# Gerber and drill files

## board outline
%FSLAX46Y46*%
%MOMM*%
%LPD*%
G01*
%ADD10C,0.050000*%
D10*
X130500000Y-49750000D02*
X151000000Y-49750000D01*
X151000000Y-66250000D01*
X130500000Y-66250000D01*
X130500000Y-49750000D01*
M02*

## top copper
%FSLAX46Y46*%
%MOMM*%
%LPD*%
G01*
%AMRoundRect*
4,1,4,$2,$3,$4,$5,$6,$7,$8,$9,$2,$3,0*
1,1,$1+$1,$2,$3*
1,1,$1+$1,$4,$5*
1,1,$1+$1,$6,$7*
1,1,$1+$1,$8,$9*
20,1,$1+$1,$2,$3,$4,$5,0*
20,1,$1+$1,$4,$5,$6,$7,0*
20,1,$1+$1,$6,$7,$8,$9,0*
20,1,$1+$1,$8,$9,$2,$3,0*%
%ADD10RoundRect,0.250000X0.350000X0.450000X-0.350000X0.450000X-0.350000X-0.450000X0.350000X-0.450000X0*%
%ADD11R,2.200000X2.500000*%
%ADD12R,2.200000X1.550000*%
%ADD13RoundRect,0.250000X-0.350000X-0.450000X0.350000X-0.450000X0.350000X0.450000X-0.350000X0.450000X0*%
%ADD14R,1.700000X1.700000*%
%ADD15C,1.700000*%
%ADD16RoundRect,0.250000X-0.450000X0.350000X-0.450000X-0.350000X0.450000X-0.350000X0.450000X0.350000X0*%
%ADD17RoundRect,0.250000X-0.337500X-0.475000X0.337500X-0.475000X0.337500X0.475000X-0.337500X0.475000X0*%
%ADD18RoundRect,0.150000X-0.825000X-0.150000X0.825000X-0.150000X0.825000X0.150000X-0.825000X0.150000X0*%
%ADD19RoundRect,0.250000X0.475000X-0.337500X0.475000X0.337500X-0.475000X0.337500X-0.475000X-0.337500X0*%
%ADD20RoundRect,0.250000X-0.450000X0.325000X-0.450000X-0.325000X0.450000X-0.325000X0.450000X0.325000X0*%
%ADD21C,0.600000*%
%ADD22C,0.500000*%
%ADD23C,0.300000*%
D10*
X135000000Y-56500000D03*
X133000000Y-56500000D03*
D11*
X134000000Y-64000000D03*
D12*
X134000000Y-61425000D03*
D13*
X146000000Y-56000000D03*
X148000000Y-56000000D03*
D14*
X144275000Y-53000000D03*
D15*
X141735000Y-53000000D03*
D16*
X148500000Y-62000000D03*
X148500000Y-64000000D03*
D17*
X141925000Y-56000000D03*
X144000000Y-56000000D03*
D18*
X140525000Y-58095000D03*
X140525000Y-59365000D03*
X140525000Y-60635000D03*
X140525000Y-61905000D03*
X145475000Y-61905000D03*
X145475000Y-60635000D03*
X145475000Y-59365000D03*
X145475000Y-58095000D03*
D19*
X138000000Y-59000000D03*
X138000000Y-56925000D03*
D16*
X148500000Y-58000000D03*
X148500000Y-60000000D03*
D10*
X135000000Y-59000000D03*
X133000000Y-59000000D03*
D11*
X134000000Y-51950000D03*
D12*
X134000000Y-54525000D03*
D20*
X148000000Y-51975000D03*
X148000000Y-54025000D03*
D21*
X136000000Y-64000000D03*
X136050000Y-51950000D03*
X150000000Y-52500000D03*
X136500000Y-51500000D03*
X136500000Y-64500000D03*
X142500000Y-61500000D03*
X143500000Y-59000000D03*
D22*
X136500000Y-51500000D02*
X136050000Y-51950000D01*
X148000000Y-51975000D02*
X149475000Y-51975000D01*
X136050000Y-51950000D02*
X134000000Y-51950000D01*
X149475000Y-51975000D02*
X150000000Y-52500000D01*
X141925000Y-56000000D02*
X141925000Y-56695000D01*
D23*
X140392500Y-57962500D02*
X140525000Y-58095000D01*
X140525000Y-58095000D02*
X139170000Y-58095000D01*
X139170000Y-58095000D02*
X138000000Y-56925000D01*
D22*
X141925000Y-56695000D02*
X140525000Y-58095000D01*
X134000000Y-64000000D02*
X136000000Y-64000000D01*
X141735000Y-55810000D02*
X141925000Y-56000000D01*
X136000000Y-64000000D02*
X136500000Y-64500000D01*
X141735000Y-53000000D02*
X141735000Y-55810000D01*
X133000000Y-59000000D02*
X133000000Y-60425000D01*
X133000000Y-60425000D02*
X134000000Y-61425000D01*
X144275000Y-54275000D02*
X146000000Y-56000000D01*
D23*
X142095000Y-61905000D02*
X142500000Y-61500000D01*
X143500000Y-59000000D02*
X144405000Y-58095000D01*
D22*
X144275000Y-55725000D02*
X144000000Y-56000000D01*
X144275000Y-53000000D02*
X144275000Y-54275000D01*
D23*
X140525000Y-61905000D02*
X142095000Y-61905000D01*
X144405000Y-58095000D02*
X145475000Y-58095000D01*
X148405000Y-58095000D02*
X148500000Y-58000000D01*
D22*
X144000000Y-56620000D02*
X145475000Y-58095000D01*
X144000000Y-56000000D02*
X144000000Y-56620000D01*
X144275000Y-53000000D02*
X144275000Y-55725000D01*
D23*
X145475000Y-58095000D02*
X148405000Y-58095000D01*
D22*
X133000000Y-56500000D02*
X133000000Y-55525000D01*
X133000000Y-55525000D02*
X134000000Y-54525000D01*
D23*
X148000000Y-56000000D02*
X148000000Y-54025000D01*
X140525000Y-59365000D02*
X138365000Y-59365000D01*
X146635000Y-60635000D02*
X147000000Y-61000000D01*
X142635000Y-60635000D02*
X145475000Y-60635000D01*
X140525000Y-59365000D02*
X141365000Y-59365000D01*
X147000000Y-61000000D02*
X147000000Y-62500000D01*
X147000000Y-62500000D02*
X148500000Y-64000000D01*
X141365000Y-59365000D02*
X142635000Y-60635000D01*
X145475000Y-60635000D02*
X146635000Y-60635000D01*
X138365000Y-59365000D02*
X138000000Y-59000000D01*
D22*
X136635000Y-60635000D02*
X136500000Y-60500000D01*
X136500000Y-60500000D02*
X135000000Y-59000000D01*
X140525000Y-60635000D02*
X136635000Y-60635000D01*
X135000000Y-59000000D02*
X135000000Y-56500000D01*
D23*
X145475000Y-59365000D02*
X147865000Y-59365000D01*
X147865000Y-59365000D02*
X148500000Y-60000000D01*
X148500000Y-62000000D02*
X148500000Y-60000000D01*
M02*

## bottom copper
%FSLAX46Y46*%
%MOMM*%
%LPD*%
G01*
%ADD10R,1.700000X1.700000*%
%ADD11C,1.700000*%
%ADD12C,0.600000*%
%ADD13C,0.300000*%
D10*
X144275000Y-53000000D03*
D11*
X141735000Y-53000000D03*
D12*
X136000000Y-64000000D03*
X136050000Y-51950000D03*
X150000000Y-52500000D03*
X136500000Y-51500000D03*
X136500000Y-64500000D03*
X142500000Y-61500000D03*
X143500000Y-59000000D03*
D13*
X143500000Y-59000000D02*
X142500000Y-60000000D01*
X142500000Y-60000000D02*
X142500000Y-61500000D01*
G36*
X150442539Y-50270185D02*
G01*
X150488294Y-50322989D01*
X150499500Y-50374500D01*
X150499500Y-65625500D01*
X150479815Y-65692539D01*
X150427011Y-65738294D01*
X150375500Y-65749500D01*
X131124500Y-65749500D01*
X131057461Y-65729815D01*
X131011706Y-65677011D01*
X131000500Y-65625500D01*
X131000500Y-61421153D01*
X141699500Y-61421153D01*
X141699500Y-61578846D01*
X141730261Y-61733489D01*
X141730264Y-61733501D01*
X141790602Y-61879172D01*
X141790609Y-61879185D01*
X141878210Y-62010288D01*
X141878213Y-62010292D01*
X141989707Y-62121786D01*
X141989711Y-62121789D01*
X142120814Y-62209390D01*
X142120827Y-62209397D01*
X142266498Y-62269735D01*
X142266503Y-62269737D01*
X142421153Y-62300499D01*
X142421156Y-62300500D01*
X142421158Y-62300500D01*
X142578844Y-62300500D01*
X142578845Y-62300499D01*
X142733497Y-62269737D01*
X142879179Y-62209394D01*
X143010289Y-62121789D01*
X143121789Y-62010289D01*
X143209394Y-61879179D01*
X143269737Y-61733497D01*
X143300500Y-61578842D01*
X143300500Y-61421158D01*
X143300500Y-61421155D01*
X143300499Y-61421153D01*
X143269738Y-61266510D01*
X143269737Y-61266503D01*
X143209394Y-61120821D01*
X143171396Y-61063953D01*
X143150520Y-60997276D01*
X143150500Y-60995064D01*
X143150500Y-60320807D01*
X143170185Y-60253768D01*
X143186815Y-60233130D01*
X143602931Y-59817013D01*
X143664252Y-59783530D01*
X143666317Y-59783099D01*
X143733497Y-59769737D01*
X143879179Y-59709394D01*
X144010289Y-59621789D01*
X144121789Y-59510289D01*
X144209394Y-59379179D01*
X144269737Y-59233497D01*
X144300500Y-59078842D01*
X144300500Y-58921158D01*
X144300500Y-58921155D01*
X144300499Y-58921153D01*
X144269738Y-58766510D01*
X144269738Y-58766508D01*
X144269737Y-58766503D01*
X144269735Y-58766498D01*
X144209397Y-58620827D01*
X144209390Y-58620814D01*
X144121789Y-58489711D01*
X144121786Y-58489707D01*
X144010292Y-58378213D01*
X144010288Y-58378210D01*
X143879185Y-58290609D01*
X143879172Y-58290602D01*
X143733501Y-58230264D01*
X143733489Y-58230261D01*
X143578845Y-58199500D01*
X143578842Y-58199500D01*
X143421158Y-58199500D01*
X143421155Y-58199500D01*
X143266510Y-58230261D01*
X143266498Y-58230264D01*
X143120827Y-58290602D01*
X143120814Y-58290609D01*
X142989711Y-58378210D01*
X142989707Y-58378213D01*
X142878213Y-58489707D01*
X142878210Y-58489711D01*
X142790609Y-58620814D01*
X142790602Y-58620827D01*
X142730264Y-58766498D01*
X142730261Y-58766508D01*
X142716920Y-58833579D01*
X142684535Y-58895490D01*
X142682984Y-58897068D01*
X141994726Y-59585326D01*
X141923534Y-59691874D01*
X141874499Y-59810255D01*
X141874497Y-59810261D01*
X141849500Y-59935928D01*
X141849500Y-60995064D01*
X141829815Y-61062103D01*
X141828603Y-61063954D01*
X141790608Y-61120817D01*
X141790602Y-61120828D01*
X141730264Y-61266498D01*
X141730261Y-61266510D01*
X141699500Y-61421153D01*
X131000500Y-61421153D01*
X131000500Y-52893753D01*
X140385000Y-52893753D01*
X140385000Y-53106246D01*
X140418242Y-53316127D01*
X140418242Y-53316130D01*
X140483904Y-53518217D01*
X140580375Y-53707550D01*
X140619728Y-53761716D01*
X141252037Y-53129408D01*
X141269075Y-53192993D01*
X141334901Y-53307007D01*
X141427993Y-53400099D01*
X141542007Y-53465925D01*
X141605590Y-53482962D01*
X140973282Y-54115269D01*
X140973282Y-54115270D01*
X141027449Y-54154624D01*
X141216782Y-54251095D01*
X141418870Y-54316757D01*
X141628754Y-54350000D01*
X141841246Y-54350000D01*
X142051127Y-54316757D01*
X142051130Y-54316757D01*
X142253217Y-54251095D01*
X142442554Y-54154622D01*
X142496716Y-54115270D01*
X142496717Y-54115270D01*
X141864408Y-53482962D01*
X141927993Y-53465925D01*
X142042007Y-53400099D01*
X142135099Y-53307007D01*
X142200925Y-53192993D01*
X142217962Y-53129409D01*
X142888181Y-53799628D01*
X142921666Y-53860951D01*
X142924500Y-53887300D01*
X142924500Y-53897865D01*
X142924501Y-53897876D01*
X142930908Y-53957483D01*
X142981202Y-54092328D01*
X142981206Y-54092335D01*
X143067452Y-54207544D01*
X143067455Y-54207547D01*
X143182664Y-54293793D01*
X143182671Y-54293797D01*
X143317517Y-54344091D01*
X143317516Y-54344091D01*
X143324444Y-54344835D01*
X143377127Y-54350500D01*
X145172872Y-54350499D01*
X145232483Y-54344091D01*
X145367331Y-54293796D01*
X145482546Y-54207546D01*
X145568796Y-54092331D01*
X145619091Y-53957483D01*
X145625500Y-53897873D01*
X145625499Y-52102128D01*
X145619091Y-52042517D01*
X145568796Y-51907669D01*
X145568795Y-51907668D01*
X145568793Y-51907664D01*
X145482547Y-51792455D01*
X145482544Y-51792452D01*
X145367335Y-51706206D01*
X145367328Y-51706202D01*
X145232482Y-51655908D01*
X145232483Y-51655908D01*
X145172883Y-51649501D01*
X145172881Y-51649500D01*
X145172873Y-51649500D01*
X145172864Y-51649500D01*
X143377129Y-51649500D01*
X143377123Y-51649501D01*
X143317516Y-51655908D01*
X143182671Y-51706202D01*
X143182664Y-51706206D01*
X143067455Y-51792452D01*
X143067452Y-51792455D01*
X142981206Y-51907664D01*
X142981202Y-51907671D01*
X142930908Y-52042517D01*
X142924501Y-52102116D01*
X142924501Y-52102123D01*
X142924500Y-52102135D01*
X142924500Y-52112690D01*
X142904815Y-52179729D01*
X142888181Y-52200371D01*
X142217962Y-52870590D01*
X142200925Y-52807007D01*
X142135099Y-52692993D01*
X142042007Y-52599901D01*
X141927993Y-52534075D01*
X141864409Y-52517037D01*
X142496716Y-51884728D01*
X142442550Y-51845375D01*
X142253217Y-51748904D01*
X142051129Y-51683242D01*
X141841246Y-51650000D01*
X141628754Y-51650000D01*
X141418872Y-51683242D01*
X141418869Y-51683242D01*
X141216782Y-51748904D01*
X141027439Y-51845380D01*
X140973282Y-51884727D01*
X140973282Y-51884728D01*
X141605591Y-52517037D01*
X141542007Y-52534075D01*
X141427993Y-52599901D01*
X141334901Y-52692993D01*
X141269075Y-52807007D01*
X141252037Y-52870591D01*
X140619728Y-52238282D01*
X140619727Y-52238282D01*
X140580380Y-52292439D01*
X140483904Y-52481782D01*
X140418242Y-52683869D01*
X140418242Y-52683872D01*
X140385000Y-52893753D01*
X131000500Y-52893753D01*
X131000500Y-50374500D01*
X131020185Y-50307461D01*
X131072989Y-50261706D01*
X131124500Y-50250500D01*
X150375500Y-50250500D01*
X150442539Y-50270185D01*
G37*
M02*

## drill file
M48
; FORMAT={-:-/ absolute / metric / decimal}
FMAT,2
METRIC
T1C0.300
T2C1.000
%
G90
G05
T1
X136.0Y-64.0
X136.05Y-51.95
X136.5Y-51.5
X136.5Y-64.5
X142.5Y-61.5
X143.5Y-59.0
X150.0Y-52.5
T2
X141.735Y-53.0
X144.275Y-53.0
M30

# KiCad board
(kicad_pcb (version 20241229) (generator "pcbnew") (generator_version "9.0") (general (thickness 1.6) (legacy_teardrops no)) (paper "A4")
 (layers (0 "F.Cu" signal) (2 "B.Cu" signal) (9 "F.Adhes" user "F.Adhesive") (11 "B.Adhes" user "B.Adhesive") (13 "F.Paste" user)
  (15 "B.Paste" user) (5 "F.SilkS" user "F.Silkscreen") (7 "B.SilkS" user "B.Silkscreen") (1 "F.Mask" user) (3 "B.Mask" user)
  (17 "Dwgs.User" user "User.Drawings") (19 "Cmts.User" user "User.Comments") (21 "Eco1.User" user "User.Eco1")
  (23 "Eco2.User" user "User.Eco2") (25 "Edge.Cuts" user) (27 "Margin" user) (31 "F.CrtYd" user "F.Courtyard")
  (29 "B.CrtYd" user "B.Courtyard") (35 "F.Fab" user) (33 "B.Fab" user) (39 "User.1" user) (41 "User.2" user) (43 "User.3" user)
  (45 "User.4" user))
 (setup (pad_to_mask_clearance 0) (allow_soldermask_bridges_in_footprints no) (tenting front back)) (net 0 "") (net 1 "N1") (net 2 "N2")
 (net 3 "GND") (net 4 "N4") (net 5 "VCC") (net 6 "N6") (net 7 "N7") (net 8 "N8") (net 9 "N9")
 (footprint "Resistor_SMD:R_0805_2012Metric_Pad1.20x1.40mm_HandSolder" (layer "F.Cu") (at 134 56.5 180)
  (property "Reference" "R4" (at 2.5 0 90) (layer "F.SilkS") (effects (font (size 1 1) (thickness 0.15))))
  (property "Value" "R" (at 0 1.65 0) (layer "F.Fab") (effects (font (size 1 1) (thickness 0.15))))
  (pad "1" smd roundrect (at -1 0 180) (size 1.2 1.4) (layers "F.Cu" "F.Mask" "F.Paste") (roundrect_rratio 0.208333) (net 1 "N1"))
  (pad "2" smd roundrect (at 1 0 180) (size 1.2 1.4) (layers "F.Cu" "F.Mask" "F.Paste") (roundrect_rratio 0.208333) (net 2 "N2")))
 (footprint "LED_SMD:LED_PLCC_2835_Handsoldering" (layer "F.Cu") (at 134 62.95 90)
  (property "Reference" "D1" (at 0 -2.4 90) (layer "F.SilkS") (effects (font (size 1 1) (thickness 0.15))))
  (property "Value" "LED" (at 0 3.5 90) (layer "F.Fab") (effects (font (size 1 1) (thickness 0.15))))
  (pad "1" smd rect (at -1.05 0 90) (size 2.5 2.2) (layers "F.Cu" "F.Mask" "F.Paste") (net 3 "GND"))
  (pad "2" smd rect (at 1.525 0 90) (size 1.55 2.2) (layers "F.Cu" "F.Mask" "F.Paste") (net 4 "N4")))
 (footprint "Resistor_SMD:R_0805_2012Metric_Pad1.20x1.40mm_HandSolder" (layer "F.Cu") (at 147 56)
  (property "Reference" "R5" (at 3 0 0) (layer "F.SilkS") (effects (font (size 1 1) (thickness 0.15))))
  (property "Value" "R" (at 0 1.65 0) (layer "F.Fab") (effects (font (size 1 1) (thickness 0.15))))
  (pad "1" smd roundrect (at -1 0) (size 1.2 1.4) (layers "F.Cu" "F.Mask" "F.Paste") (roundrect_rratio 0.208333) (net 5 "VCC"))
  (pad "2" smd roundrect (at 1 0) (size 1.2 1.4) (layers "F.Cu" "F.Mask" "F.Paste") (roundrect_rratio 0.208333) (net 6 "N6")))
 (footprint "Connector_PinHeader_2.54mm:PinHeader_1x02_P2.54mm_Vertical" (layer "F.Cu") (at 144.275 53 -90)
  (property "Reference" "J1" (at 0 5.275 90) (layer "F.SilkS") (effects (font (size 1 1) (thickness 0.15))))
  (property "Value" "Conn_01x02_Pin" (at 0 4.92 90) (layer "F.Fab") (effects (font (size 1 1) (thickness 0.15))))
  (pad "1" thru_hole rect (at 0 0 270) (size 1.7 1.7) (drill 1) (layers "*.Cu" "*.Mask") (remove_unused_layers no) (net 5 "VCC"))
  (pad "2" thru_hole circle (at 0 2.54 270) (size 1.7 1.7) (drill 1) (layers "*.Cu" "*.Mask") (remove_unused_layers no) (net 3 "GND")))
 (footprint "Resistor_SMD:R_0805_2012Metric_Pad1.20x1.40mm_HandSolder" (layer "F.Cu") (at 148.5 63 -90)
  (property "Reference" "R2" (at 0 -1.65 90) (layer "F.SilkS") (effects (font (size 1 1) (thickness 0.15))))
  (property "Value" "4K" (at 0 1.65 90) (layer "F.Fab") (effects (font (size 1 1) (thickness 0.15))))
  (pad "1" smd roundrect (at -1 0 270) (size 1.2 1.4) (layers "F.Cu" "F.Mask" "F.Paste") (roundrect_rratio 0.208333) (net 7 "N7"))
  (pad "2" smd roundrect (at 1 0 270) (size 1.2 1.4) (layers "F.Cu" "F.Mask" "F.Paste") (roundrect_rratio 0.208333) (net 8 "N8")))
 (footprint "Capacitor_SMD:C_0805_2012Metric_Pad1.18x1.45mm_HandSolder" (layer "F.Cu") (at 142.9625 56)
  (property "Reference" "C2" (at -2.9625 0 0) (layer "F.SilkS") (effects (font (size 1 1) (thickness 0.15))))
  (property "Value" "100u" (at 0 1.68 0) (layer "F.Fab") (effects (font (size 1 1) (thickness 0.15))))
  (pad "1" smd roundrect (at -1.0375 0) (size 1.175 1.45) (layers "F.Cu" "F.Mask" "F.Paste") (roundrect_rratio 0.212766) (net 3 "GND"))
  (pad "2" smd roundrect (at 1.0375 0) (size 1.175 1.45) (layers "F.Cu" "F.Mask" "F.Paste") (roundrect_rratio 0.212766) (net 5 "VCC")))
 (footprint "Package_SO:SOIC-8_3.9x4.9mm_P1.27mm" (layer "F.Cu") (at 143 60)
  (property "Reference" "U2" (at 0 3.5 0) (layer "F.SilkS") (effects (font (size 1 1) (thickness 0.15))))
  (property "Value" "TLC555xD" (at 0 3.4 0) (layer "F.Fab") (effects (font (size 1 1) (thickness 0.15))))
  (pad "1" smd roundrect (at -2.475 -1.905) (size 1.95 0.6) (layers "F.Cu" "F.Mask" "F.Paste") (roundrect_rratio 0.25) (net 3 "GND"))
  (pad "2" smd roundrect (at -2.475 -0.635) (size 1.95 0.6) (layers "F.Cu" "F.Mask" "F.Paste") (roundrect_rratio 0.25) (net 8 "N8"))
  (pad "3" smd roundrect (at -2.475 0.635) (size 1.95 0.6) (layers "F.Cu" "F.Mask" "F.Paste") (roundrect_rratio 0.25) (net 1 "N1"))
  (pad "4" smd roundrect (at -2.475 1.905) (size 1.95 0.6) (layers "F.Cu" "F.Mask" "F.Paste") (roundrect_rratio 0.25) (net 5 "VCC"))
  (pad "5" smd roundrect (at 2.475 1.905) (size 1.95 0.6) (layers "F.Cu" "F.Mask" "F.Paste") (roundrect_rratio 0.25) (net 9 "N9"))
  (pad "6" smd roundrect (at 2.475 0.635) (size 1.95 0.6) (layers "F.Cu" "F.Mask" "F.Paste") (roundrect_rratio 0.25) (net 8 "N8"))
  (pad "7" smd roundrect (at 2.475 -0.635) (size 1.95 0.6) (layers "F.Cu" "F.Mask" "F.Paste") (roundrect_rratio 0.25) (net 7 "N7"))
  (pad "8" smd roundrect (at 2.475 -1.905) (size 1.95 0.6) (layers "F.Cu" "F.Mask" "F.Paste") (roundrect_rratio 0.25) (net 5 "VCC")))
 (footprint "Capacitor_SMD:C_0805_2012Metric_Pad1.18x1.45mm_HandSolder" (layer "F.Cu") (at 138 57.9625 90)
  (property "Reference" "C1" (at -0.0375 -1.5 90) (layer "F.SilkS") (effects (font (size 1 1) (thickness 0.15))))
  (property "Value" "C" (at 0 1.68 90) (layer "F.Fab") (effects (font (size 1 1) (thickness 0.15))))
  (pad "1" smd roundrect (at -1.0375 0 90) (size 1.175 1.45) (layers "F.Cu" "F.Mask" "F.Paste") (roundrect_rratio 0.212766) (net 8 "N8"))
  (pad "2" smd roundrect (at 1.0375 0 90) (size 1.175 1.45) (layers "F.Cu" "F.Mask" "F.Paste") (roundrect_rratio 0.212766) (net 3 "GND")))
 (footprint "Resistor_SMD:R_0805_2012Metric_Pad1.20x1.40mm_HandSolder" (layer "F.Cu") (at 148.5 59 -90)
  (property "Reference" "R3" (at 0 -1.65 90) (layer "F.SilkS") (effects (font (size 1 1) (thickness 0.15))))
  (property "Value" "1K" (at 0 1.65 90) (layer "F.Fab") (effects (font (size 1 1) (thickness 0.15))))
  (pad "1" smd roundrect (at -1 0 270) (size 1.2 1.4) (layers "F.Cu" "F.Mask" "F.Paste") (roundrect_rratio 0.208333) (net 5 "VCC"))
  (pad "2" smd roundrect (at 1 0 270) (size 1.2 1.4) (layers "F.Cu" "F.Mask" "F.Paste") (roundrect_rratio 0.208333) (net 7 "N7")))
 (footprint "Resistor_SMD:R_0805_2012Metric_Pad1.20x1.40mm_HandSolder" (layer "F.Cu") (at 134 59 180)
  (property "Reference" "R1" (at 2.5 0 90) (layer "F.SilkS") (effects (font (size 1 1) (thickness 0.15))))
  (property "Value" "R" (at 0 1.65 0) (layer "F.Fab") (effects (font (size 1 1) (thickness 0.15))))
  (pad "1" smd roundrect (at -1 0 180) (size 1.2 1.4) (layers "F.Cu" "F.Mask" "F.Paste") (roundrect_rratio 0.208333) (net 1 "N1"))
  (pad "2" smd roundrect (at 1 0 180) (size 1.2 1.4) (layers "F.Cu" "F.Mask" "F.Paste") (roundrect_rratio 0.208333) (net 4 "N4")))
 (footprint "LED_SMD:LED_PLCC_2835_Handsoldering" (layer "F.Cu") (at 134 53 -90)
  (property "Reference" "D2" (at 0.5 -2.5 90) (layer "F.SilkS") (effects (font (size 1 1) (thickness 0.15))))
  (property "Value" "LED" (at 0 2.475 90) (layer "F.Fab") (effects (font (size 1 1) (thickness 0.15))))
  (pad "1" smd rect (at -1.05 0 270) (size 2.5 2.2) (layers "F.Cu" "F.Mask" "F.Paste") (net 3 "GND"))
  (pad "2" smd rect (at 1.525 0 270) (size 1.55 2.2) (layers "F.Cu" "F.Mask" "F.Paste") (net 2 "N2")))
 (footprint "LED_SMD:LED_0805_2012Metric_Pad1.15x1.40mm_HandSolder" (layer "F.Cu") (at 148 53 -90)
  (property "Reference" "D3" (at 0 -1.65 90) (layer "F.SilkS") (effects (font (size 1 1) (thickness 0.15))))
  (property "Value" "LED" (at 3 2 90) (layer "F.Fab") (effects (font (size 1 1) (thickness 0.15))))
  (pad "1" smd roundrect (at -1.025 0 270) (size 1.15 1.4) (layers "F.Cu" "F.Mask" "F.Paste") (roundrect_rratio 0.217391) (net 3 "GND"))
  (pad "2" smd roundrect (at 1.025 0 270) (size 1.15 1.4) (layers "F.Cu" "F.Mask" "F.Paste") (roundrect_rratio 0.217391) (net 6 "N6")))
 (gr_rect (start 130.5 49.75) (end 151 66.25) (stroke (width 0.05) (type default)) (fill no) (layer "Edge.Cuts"))
 (segment (start 136.5 51.5) (end 136.05 51.95) (width 0.5) (layer "F.Cu") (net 3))
 (segment (start 148 51.975) (end 149.475 51.975) (width 0.5) (layer "F.Cu") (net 3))
 (segment (start 136.05 51.95) (end 134 51.95) (width 0.5) (layer "F.Cu") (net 3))
 (segment (start 149.475 51.975) (end 150 52.5) (width 0.5) (layer "F.Cu") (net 3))
 (segment (start 141.925 56) (end 141.925 56.695) (width 0.5) (layer "F.Cu") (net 3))
 (segment (start 140.3925 57.9625) (end 140.525 58.095) (width 0.3) (layer "F.Cu") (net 3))
 (segment (start 140.525 58.095) (end 139.17 58.095) (width 0.3) (layer "F.Cu") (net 3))
 (segment (start 139.17 58.095) (end 138 56.925) (width 0.3) (layer "F.Cu") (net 3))
 (segment (start 141.925 56.695) (end 140.525 58.095) (width 0.5) (layer "F.Cu") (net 3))
 (segment (start 134 64) (end 136 64) (width 0.5) (layer "F.Cu") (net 3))
 (segment (start 141.735 55.81) (end 141.925 56) (width 0.5) (layer "F.Cu") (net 3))
 (segment (start 136 64) (end 136.5 64.5) (width 0.5) (layer "F.Cu") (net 3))
 (segment (start 141.735 53) (end 141.735 55.81) (width 0.5) (layer "F.Cu") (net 3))
 (via (at 136 64) (size 0.6) (drill 0.3) (layers "F.Cu" "B.Cu") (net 3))
 (via (at 136.05 51.95) (size 0.6) (drill 0.3) (layers "F.Cu" "B.Cu") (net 3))
 (via (at 150 52.5) (size 0.6) (drill 0.3) (layers "F.Cu" "B.Cu") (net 3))
 (via (at 136.5 51.5) (size 0.6) (drill 0.3) (layers "F.Cu" "B.Cu") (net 3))
 (via (at 136.5 64.5) (size 0.6) (drill 0.3) (layers "F.Cu" "B.Cu") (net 3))
 (segment (start 133 59) (end 133 60.425) (width 0.5) (layer "F.Cu") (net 4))
 (segment (start 133 60.425) (end 134 61.425) (width 0.5) (layer "F.Cu") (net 4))
 (segment (start 144.275 54.275) (end 146 56) (width 0.5) (layer "F.Cu") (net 5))
 (segment (start 142.095 61.905) (end 142.5 61.5) (width 0.3) (layer "F.Cu") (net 5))
 (segment (start 143.5 59) (end 144.405 58.095) (width 0.3) (layer "F.Cu") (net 5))
 (segment (start 144.275 55.725) (end 144 56) (width 0.5) (layer "F.Cu") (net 5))
 (segment (start 144.275 53) (end 144.275 54.275) (width 0.5) (layer "F.Cu") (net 5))
 (segment (start 140.525 61.905) (end 142.095 61.905) (width 0.3) (layer "F.Cu") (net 5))
 (segment (start 144.405 58.095) (end 145.475 58.095) (width 0.3) (layer "F.Cu") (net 5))
 (segment (start 148.405 58.095) (end 148.5 58) (width 0.3) (layer "F.Cu") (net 5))
 (segment (start 144 56.62) (end 145.475 58.095) (width 0.5) (layer "F.Cu") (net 5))
 (segment (start 144 56) (end 144 56.62) (width 0.5) (layer "F.Cu") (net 5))
 (segment (start 144.275 53) (end 144.275 55.725) (width 0.5) (layer "F.Cu") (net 5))
 (segment (start 145.475 58.095) (end 148.405 58.095) (width 0.3) (layer "F.Cu") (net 5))
 (via (at 142.5 61.5) (size 0.6) (drill 0.3) (layers "F.Cu" "B.Cu") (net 5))
 (via (at 143.5 59) (size 0.6) (drill 0.3) (layers "F.Cu" "B.Cu") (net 5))
 (segment (start 143.5 59) (end 142.5 60) (width 0.3) (layer "B.Cu") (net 5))
 (segment (start 142.5 60) (end 142.5 61.5) (width 0.3) (layer "B.Cu") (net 5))
 (segment (start 133 56.5) (end 133 55.525) (width 0.5) (layer "F.Cu") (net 2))
 (segment (start 133 55.525) (end 134 54.525) (width 0.5) (layer "F.Cu") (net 2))
 (segment (start 148 56) (end 148 54.025) (width 0.3) (layer "F.Cu") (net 6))
 (segment (start 140.525 59.365) (end 138.365 59.365) (width 0.3) (layer "F.Cu") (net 8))
 (segment (start 146.635 60.635) (end 147 61) (width 0.3) (layer "F.Cu") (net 8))
 (segment (start 142.635 60.635) (end 145.475 60.635) (width 0.3) (layer "F.Cu") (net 8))
 (segment (start 140.525 59.365) (end 141.365 59.365) (width 0.3) (layer "F.Cu") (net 8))
 (segment (start 147 61) (end 147 62.5) (width 0.3) (layer "F.Cu") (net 8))
 (segment (start 147 62.5) (end 148.5 64) (width 0.3) (layer "F.Cu") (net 8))
 (segment (start 141.365 59.365) (end 142.635 60.635) (width 0.3) (layer "F.Cu") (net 8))
 (segment (start 145.475 60.635) (end 146.635 60.635) (width 0.3) (layer "F.Cu") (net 8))
 (segment (start 138.365 59.365) (end 138 59) (width 0.3) (layer "F.Cu") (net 8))
 (segment (start 136.635 60.635) (end 136.5 60.5) (width 0.5) (layer "F.Cu") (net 1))
 (segment (start 136.5 60.5) (end 135 59) (width 0.5) (layer "F.Cu") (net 1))
 (segment (start 140.525 60.635) (end 136.635 60.635) (width 0.5) (layer "F.Cu") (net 1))
 (segment (start 135 59) (end 135 56.5) (width 0.5) (layer "F.Cu") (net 1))
 (segment (start 145.475 59.365) (end 147.865 59.365) (width 0.3) (layer "F.Cu") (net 7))
 (segment (start 147.865 59.365) (end 148.5 60) (width 0.3) (layer "F.Cu") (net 7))
 (segment (start 148.5 62) (end 148.5 60) (width 0.3) (layer "F.Cu") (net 7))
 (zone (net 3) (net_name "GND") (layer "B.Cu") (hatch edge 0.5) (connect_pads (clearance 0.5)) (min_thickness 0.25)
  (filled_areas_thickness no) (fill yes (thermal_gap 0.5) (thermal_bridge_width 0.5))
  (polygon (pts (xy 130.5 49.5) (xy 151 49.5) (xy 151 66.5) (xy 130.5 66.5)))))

